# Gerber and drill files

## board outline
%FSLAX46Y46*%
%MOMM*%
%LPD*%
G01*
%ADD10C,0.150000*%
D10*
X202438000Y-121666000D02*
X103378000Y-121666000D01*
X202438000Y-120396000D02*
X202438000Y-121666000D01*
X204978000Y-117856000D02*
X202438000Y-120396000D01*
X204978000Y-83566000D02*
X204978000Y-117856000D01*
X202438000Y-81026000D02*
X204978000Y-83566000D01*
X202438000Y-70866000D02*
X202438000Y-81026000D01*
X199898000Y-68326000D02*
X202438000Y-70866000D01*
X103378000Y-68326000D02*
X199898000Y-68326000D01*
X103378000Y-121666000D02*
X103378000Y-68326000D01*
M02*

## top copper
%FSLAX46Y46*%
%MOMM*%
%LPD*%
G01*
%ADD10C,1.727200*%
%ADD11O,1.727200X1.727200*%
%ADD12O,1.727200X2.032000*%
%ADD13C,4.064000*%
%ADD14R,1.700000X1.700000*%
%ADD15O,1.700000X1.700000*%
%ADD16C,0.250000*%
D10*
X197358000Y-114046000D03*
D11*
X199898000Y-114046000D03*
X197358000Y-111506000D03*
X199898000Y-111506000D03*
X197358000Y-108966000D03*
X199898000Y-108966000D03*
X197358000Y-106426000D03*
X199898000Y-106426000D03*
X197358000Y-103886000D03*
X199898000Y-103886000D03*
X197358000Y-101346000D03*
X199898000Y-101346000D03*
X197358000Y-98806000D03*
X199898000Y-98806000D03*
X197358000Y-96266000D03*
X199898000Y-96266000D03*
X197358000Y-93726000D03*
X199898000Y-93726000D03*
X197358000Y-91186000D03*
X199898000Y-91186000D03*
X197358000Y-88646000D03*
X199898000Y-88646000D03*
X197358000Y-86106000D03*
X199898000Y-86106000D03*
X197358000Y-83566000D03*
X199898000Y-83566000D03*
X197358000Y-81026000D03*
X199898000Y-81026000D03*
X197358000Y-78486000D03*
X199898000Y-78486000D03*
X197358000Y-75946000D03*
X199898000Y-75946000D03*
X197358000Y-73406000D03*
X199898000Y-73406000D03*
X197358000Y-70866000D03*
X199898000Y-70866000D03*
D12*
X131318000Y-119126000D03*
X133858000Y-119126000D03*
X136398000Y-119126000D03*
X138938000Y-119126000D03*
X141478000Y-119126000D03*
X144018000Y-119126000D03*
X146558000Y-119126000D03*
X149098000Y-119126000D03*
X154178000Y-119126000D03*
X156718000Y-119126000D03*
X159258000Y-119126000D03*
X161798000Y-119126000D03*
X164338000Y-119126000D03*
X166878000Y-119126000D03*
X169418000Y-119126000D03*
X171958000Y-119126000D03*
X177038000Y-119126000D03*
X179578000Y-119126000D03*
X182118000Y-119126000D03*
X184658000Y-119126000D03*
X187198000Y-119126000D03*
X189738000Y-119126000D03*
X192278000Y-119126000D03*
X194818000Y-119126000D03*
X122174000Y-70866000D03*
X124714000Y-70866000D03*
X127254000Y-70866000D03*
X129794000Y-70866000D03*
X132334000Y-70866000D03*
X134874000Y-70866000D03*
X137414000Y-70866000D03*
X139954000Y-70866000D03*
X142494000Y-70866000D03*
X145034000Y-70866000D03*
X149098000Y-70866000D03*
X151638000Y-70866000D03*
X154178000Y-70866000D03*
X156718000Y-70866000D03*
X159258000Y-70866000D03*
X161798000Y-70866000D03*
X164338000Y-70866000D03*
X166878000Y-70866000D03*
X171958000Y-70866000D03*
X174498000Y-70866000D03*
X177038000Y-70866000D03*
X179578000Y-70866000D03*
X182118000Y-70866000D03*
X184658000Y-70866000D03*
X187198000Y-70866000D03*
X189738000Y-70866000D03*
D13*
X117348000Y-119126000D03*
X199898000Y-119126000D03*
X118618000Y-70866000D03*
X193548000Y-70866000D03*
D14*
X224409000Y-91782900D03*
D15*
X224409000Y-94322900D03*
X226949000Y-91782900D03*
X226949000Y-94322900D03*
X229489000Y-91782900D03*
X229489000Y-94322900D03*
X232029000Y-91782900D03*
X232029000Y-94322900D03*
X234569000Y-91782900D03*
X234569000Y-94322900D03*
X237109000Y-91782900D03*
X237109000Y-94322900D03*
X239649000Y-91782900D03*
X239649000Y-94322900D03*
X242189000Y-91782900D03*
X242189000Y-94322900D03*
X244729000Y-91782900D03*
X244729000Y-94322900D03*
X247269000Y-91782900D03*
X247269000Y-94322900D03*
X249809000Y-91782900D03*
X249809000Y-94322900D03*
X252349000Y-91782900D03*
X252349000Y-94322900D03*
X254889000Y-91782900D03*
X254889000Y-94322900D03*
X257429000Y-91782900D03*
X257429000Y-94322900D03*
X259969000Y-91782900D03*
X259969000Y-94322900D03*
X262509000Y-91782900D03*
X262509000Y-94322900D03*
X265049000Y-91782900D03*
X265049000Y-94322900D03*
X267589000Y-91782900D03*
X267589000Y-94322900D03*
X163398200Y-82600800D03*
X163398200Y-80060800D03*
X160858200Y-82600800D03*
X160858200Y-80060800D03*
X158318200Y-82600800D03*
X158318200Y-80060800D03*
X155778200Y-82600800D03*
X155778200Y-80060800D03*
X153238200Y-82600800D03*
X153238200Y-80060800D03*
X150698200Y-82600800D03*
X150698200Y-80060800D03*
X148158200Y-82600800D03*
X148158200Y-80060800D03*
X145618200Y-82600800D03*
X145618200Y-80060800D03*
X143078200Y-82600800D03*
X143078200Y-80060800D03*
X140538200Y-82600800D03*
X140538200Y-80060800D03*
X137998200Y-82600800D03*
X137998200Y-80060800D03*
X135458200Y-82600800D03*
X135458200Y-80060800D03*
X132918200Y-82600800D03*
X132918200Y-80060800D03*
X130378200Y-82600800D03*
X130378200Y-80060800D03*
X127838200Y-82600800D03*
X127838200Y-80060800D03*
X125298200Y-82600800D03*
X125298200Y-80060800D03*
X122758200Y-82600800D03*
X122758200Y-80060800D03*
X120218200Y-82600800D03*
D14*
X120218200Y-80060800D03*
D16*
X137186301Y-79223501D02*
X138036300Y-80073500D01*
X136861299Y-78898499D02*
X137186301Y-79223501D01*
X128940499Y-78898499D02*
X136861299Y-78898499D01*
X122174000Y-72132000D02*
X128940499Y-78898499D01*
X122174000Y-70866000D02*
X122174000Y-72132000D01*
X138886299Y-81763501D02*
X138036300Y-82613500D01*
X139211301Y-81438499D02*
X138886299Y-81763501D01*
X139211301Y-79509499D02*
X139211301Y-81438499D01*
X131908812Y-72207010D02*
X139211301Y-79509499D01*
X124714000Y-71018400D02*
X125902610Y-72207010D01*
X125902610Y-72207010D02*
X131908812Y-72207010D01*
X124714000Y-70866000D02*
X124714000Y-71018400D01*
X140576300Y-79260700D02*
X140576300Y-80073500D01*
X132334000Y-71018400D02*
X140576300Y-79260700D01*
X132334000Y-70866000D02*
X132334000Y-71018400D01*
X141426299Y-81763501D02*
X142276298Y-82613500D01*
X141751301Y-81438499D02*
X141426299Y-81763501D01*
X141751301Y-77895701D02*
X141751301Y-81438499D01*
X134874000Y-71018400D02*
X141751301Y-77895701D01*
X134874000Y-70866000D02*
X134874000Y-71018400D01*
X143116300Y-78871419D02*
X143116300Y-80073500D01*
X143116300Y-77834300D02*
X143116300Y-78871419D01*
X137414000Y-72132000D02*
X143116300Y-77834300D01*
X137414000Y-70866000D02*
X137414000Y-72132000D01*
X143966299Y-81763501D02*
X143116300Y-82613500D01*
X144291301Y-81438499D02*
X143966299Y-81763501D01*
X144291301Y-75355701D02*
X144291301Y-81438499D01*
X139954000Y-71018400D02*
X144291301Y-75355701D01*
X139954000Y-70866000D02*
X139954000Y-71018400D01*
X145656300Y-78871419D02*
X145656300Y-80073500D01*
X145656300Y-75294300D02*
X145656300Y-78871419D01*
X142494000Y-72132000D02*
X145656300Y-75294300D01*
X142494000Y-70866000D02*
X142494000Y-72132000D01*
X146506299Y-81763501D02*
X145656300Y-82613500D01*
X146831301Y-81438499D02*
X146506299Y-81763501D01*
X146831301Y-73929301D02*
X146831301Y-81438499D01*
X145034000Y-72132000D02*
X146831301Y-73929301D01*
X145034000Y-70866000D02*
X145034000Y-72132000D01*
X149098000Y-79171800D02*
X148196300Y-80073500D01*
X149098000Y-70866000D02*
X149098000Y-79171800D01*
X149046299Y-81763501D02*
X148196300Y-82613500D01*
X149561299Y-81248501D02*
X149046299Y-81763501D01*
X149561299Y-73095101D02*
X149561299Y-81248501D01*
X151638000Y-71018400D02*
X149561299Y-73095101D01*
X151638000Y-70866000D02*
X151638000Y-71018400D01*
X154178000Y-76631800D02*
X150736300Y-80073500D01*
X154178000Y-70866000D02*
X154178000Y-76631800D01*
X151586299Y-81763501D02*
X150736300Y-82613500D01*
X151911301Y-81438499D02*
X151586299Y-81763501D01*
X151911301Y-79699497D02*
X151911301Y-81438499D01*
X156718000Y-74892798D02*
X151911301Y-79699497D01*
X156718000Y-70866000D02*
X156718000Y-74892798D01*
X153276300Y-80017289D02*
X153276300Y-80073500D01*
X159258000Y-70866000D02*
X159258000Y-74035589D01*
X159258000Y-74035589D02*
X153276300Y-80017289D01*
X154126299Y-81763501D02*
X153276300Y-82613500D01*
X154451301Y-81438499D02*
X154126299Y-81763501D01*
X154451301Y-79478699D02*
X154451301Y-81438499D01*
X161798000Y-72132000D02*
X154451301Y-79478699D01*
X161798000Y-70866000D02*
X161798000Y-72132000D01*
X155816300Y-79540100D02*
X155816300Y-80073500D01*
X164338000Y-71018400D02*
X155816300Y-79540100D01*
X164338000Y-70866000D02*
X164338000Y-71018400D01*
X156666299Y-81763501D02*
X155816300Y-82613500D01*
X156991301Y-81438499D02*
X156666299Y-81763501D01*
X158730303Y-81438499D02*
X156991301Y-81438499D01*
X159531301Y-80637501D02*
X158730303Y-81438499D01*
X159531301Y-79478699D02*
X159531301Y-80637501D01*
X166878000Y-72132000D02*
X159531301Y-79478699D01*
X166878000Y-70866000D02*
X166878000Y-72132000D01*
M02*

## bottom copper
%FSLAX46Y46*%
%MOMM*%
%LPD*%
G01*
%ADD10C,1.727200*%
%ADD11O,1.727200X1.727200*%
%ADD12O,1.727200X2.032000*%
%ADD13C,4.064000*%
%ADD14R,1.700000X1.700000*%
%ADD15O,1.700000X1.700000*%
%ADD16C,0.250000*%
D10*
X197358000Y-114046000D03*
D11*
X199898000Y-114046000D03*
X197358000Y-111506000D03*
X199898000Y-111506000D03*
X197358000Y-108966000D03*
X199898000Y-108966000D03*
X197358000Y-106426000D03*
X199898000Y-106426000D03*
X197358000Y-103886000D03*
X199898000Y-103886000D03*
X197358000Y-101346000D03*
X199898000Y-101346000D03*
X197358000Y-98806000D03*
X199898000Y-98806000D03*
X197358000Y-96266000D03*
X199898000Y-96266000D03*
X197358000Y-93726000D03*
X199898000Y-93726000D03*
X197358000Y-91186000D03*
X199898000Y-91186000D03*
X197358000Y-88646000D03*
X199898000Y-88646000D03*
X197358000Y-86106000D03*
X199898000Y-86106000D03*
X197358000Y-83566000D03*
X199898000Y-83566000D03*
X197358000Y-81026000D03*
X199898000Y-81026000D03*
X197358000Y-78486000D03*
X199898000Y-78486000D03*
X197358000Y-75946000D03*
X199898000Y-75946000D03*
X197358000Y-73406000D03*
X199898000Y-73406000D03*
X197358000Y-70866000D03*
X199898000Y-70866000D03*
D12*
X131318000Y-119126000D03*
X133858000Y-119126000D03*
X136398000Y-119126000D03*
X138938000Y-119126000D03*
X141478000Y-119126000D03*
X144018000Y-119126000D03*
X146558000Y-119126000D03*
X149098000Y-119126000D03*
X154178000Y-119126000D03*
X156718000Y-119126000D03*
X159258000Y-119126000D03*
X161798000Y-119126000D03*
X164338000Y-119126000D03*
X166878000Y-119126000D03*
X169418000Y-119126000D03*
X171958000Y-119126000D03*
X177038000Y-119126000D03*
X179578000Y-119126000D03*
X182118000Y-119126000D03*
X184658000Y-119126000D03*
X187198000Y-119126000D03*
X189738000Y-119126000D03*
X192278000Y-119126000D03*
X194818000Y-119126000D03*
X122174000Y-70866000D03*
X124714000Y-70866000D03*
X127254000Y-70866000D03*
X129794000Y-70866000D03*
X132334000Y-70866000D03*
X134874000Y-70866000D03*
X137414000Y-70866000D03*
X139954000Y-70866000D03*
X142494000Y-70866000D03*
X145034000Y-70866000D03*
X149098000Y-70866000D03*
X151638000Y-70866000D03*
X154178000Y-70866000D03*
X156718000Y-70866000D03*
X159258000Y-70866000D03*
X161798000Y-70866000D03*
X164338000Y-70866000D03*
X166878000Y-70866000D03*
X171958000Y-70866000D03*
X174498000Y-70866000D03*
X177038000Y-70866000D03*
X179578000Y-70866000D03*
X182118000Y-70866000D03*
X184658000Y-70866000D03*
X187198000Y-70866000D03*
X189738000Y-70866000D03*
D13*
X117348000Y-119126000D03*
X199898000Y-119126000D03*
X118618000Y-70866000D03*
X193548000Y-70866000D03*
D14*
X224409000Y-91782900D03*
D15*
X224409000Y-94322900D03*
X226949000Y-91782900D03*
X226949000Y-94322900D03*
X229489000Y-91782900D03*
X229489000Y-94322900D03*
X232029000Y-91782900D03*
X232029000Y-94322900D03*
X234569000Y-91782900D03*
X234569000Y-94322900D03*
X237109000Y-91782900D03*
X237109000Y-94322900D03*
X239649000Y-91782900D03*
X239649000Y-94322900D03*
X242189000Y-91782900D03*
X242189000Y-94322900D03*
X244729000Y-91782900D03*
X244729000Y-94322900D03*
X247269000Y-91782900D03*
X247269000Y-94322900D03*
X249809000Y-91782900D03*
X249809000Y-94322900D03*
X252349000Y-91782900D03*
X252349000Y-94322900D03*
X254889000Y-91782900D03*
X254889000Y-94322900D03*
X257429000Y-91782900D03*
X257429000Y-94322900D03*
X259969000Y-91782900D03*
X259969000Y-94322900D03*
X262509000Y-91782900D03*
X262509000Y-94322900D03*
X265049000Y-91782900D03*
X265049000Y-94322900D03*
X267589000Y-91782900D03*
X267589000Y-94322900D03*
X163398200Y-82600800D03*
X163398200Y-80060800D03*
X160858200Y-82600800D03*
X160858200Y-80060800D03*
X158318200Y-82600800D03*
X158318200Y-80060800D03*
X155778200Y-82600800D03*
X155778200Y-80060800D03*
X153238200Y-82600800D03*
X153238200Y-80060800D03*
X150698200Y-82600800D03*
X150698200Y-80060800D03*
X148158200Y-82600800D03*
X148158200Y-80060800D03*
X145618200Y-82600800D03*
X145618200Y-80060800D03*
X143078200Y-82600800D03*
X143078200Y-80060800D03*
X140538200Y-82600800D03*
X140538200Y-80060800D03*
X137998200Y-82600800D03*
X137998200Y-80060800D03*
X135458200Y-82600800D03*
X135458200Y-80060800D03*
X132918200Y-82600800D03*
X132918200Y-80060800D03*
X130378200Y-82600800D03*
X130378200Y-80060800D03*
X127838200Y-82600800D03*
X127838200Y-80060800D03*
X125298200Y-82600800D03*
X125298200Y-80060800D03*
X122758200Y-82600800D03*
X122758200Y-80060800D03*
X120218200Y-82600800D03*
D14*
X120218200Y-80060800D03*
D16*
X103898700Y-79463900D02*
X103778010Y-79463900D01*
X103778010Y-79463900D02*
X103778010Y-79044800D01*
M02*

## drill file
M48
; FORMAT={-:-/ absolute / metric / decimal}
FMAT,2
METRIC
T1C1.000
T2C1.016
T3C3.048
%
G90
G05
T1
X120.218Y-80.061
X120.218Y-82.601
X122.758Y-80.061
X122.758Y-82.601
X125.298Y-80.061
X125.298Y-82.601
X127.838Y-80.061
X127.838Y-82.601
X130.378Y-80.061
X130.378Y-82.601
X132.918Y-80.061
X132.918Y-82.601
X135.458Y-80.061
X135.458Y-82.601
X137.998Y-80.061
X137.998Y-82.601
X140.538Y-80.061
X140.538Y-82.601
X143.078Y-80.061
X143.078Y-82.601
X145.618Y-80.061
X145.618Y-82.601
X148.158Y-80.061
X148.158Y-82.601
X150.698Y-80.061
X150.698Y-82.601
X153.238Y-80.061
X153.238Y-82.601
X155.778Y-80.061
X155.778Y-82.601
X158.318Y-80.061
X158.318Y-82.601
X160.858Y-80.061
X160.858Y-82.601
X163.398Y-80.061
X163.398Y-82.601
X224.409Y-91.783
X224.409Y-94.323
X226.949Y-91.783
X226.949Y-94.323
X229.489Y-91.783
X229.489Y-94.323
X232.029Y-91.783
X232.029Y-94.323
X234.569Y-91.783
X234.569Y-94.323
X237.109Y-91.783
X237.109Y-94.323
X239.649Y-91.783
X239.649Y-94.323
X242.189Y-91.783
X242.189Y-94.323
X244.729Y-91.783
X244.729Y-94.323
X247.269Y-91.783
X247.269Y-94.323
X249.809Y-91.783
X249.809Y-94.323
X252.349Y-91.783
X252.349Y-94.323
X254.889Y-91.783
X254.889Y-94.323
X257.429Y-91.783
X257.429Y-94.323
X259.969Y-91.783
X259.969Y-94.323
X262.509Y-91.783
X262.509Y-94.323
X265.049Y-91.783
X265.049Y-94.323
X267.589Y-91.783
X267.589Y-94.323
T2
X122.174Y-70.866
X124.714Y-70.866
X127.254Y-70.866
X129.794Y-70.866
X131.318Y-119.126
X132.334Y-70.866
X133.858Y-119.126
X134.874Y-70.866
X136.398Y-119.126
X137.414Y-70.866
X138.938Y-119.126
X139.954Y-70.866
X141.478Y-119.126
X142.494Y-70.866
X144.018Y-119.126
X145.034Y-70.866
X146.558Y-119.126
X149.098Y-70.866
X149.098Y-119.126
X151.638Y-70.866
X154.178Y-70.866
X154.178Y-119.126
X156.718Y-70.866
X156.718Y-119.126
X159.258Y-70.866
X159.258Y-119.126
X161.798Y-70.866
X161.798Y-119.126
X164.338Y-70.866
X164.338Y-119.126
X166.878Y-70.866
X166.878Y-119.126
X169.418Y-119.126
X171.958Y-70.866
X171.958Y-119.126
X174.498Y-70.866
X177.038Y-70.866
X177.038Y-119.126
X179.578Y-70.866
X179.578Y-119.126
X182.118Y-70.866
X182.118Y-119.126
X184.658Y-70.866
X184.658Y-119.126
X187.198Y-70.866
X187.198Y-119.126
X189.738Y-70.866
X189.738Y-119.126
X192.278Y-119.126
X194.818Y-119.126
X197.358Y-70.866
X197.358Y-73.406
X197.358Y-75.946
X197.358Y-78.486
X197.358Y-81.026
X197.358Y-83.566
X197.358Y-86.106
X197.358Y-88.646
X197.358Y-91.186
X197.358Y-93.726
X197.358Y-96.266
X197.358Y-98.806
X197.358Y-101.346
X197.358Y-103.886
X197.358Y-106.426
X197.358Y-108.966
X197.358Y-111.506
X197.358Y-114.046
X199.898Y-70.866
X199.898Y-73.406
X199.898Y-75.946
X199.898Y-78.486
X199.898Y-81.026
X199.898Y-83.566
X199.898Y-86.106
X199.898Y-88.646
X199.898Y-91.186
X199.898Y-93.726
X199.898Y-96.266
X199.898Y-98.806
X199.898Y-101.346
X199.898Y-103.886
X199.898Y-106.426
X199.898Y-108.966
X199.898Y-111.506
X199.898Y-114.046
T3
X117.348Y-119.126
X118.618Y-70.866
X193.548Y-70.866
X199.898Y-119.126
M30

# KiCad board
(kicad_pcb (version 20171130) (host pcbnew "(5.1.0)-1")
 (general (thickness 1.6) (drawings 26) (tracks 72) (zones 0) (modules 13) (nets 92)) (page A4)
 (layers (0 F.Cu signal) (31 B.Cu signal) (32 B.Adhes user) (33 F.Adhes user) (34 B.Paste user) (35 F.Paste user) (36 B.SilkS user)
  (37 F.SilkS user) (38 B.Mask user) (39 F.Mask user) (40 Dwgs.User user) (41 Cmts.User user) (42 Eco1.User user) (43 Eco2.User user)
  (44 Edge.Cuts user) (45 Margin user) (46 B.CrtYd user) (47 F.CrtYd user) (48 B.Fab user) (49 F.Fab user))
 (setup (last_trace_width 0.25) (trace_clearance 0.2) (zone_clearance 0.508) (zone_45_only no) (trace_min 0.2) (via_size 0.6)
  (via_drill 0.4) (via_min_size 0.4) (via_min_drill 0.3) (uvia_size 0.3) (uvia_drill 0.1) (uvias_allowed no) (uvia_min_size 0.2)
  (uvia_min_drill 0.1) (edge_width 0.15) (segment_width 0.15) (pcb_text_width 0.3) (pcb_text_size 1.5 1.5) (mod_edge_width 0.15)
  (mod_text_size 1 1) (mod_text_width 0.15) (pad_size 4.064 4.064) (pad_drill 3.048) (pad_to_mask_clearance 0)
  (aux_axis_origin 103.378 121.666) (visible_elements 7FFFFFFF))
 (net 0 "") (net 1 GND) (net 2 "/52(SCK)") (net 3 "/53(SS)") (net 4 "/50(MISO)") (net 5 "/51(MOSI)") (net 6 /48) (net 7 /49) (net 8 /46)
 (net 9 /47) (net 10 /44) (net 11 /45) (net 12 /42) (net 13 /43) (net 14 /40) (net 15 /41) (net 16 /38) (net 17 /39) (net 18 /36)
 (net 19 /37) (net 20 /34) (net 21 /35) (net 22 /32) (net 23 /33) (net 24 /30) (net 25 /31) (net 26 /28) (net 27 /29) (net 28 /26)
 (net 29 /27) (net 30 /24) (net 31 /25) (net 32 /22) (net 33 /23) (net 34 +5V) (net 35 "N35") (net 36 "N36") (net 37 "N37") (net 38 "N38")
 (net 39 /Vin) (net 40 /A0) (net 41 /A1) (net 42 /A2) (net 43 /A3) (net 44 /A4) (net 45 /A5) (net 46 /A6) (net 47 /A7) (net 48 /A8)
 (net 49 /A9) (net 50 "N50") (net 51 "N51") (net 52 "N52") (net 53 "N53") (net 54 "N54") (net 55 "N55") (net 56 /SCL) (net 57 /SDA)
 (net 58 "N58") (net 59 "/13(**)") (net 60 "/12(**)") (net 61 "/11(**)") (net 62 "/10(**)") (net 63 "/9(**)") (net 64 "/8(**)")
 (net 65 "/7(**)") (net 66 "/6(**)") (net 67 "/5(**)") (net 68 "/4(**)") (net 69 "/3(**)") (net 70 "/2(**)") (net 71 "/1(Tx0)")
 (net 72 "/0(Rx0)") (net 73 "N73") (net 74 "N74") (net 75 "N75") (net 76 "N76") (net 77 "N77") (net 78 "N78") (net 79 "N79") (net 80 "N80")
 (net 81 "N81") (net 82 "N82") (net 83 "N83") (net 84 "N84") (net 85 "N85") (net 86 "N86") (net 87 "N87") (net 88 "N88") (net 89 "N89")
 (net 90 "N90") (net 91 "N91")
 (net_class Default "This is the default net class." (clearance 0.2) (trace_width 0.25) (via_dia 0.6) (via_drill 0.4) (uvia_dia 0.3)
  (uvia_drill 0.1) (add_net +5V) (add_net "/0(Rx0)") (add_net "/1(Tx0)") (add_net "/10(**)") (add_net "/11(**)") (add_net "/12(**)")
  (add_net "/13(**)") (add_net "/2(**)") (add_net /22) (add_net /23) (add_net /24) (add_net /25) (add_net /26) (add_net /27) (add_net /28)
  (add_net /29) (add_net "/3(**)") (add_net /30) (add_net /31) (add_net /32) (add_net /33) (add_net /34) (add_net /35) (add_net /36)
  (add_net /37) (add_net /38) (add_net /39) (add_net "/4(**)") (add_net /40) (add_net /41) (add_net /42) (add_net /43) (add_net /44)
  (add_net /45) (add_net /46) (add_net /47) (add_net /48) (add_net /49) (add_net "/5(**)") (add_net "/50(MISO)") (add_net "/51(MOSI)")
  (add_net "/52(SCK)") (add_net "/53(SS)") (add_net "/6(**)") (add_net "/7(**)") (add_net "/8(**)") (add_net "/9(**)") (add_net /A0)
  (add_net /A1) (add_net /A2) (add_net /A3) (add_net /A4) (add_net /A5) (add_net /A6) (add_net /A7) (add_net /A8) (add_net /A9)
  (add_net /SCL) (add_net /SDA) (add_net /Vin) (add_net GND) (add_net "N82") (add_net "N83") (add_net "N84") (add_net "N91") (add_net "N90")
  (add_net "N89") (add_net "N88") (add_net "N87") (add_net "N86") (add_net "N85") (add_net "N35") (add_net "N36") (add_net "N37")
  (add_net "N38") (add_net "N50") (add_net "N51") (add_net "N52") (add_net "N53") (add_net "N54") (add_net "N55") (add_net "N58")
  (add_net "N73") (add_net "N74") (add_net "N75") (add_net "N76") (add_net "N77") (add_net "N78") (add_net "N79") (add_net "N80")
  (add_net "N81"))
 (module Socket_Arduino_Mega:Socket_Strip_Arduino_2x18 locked (layer F.Cu) (at 197.358 114.046 90)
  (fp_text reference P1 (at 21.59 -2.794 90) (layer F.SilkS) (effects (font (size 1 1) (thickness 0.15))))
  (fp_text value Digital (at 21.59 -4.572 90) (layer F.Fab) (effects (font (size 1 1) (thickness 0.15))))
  (pad 1 thru_hole circle (at 0 0 90) (size 1.7272 1.7272) (drill 1.016) (layers *.Cu *.Mask F.SilkS) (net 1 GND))
  (pad 2 thru_hole oval (at 0 2.54 90) (size 1.7272 1.7272) (drill 1.016) (layers *.Cu *.Mask F.SilkS) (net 1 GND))
  (pad 3 thru_hole oval (at 2.54 0 90) (size 1.7272 1.7272) (drill 1.016) (layers *.Cu *.Mask F.SilkS) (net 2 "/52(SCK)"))
  (pad 4 thru_hole oval (at 2.54 2.54 90) (size 1.7272 1.7272) (drill 1.016) (layers *.Cu *.Mask F.SilkS) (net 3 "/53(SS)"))
  (pad 5 thru_hole oval (at 5.08 0 90) (size 1.7272 1.7272) (drill 1.016) (layers *.Cu *.Mask F.SilkS) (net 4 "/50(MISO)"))
  (pad 6 thru_hole oval (at 5.08 2.54 90) (size 1.7272 1.7272) (drill 1.016) (layers *.Cu *.Mask F.SilkS) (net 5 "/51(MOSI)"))
  (pad 7 thru_hole oval (at 7.62 0 90) (size 1.7272 1.7272) (drill 1.016) (layers *.Cu *.Mask F.SilkS) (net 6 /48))
  (pad 8 thru_hole oval (at 7.62 2.54 90) (size 1.7272 1.7272) (drill 1.016) (layers *.Cu *.Mask F.SilkS) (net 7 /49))
  (pad 9 thru_hole oval (at 10.16 0 90) (size 1.7272 1.7272) (drill 1.016) (layers *.Cu *.Mask F.SilkS) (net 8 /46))
  (pad 10 thru_hole oval (at 10.16 2.54 90) (size 1.7272 1.7272) (drill 1.016) (layers *.Cu *.Mask F.SilkS) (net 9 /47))
  (pad 11 thru_hole oval (at 12.7 0 90) (size 1.7272 1.7272) (drill 1.016) (layers *.Cu *.Mask F.SilkS) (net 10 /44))
  (pad 12 thru_hole oval (at 12.7 2.54 90) (size 1.7272 1.7272) (drill 1.016) (layers *.Cu *.Mask F.SilkS) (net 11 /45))
  (pad 13 thru_hole oval (at 15.24 0 90) (size 1.7272 1.7272) (drill 1.016) (layers *.Cu *.Mask F.SilkS) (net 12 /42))
  (pad 14 thru_hole oval (at 15.24 2.54 90) (size 1.7272 1.7272) (drill 1.016) (layers *.Cu *.Mask F.SilkS) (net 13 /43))
  (pad 15 thru_hole oval (at 17.78 0 90) (size 1.7272 1.7272) (drill 1.016) (layers *.Cu *.Mask F.SilkS) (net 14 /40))
  (pad 16 thru_hole oval (at 17.78 2.54 90) (size 1.7272 1.7272) (drill 1.016) (layers *.Cu *.Mask F.SilkS) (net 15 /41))
  (pad 17 thru_hole oval (at 20.32 0 90) (size 1.7272 1.7272) (drill 1.016) (layers *.Cu *.Mask F.SilkS) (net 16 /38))
  (pad 18 thru_hole oval (at 20.32 2.54 90) (size 1.7272 1.7272) (drill 1.016) (layers *.Cu *.Mask F.SilkS) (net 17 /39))
  (pad 19 thru_hole oval (at 22.86 0 90) (size 1.7272 1.7272) (drill 1.016) (layers *.Cu *.Mask F.SilkS) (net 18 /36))
  (pad 20 thru_hole oval (at 22.86 2.54 90) (size 1.7272 1.7272) (drill 1.016) (layers *.Cu *.Mask F.SilkS) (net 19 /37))
  (pad 21 thru_hole oval (at 25.4 0 90) (size 1.7272 1.7272) (drill 1.016) (layers *.Cu *.Mask F.SilkS) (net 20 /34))
  (pad 22 thru_hole oval (at 25.4 2.54 90) (size 1.7272 1.7272) (drill 1.016) (layers *.Cu *.Mask F.SilkS) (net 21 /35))
  (pad 23 thru_hole oval (at 27.94 0 90) (size 1.7272 1.7272) (drill 1.016) (layers *.Cu *.Mask F.SilkS) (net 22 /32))
  (pad 24 thru_hole oval (at 27.94 2.54 90) (size 1.7272 1.7272) (drill 1.016) (layers *.Cu *.Mask F.SilkS) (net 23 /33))
  (pad 25 thru_hole oval (at 30.48 0 90) (size 1.7272 1.7272) (drill 1.016) (layers *.Cu *.Mask F.SilkS) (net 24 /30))
  (pad 26 thru_hole oval (at 30.48 2.54 90) (size 1.7272 1.7272) (drill 1.016) (layers *.Cu *.Mask F.SilkS) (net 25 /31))
  (pad 27 thru_hole oval (at 33.02 0 90) (size 1.7272 1.7272) (drill 1.016) (layers *.Cu *.Mask F.SilkS) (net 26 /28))
  (pad 28 thru_hole oval (at 33.02 2.54 90) (size 1.7272 1.7272) (drill 1.016) (layers *.Cu *.Mask F.SilkS) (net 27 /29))
  (pad 29 thru_hole oval (at 35.56 0 90) (size 1.7272 1.7272) (drill 1.016) (layers *.Cu *.Mask F.SilkS) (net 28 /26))
  (pad 30 thru_hole oval (at 35.56 2.54 90) (size 1.7272 1.7272) (drill 1.016) (layers *.Cu *.Mask F.SilkS) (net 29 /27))
  (pad 31 thru_hole oval (at 38.1 0 90) (size 1.7272 1.7272) (drill 1.016) (layers *.Cu *.Mask F.SilkS) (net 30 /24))
  (pad 32 thru_hole oval (at 38.1 2.54 90) (size 1.7272 1.7272) (drill 1.016) (layers *.Cu *.Mask F.SilkS) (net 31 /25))
  (pad 33 thru_hole oval (at 40.64 0 90) (size 1.7272 1.7272) (drill 1.016) (layers *.Cu *.Mask F.SilkS) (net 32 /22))
  (pad 34 thru_hole oval (at 40.64 2.54 90) (size 1.7272 1.7272) (drill 1.016) (layers *.Cu *.Mask F.SilkS) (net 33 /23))
  (pad 35 thru_hole oval (at 43.18 0 90) (size 1.7272 1.7272) (drill 1.016) (layers *.Cu *.Mask F.SilkS) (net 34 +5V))
  (pad 36 thru_hole oval (at 43.18 2.54 90) (size 1.7272 1.7272) (drill 1.016) (layers *.Cu *.Mask F.SilkS) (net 34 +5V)))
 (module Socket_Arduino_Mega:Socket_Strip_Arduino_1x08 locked (layer F.Cu) (at 131.318 119.126)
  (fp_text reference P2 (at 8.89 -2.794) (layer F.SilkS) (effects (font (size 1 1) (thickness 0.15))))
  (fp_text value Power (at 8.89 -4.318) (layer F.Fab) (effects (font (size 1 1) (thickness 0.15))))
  (pad 1 thru_hole oval (at 0 0) (size 1.7272 2.032) (drill 1.016) (layers *.Cu *.Mask F.SilkS) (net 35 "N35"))
  (pad 2 thru_hole oval (at 2.54 0) (size 1.7272 2.032) (drill 1.016) (layers *.Cu *.Mask F.SilkS) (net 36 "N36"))
  (pad 3 thru_hole oval (at 5.08 0) (size 1.7272 2.032) (drill 1.016) (layers *.Cu *.Mask F.SilkS) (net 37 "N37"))
  (pad 4 thru_hole oval (at 7.62 0) (size 1.7272 2.032) (drill 1.016) (layers *.Cu *.Mask F.SilkS) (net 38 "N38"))
  (pad 5 thru_hole oval (at 10.16 0) (size 1.7272 2.032) (drill 1.016) (layers *.Cu *.Mask F.SilkS) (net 34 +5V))
  (pad 6 thru_hole oval (at 12.7 0) (size 1.7272 2.032) (drill 1.016) (layers *.Cu *.Mask F.SilkS) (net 1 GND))
  (pad 7 thru_hole oval (at 15.24 0) (size 1.7272 2.032) (drill 1.016) (layers *.Cu *.Mask F.SilkS) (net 1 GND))
  (pad 8 thru_hole oval (at 17.78 0) (size 1.7272 2.032) (drill 1.016) (layers *.Cu *.Mask F.SilkS) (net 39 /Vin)))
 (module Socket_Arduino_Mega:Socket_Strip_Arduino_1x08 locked (layer F.Cu) (at 154.178 119.126)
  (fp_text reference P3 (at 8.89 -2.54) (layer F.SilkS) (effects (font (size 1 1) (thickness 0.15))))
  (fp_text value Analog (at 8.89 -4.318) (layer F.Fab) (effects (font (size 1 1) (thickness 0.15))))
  (pad 1 thru_hole oval (at 0 0) (size 1.7272 2.032) (drill 1.016) (layers *.Cu *.Mask F.SilkS) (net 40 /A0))
  (pad 2 thru_hole oval (at 2.54 0) (size 1.7272 2.032) (drill 1.016) (layers *.Cu *.Mask F.SilkS) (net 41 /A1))
  (pad 3 thru_hole oval (at 5.08 0) (size 1.7272 2.032) (drill 1.016) (layers *.Cu *.Mask F.SilkS) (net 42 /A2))
  (pad 4 thru_hole oval (at 7.62 0) (size 1.7272 2.032) (drill 1.016) (layers *.Cu *.Mask F.SilkS) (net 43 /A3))
  (pad 5 thru_hole oval (at 10.16 0) (size 1.7272 2.032) (drill 1.016) (layers *.Cu *.Mask F.SilkS) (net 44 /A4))
  (pad 6 thru_hole oval (at 12.7 0) (size 1.7272 2.032) (drill 1.016) (layers *.Cu *.Mask F.SilkS) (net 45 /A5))
  (pad 7 thru_hole oval (at 15.24 0) (size 1.7272 2.032) (drill 1.016) (layers *.Cu *.Mask F.SilkS) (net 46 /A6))
  (pad 8 thru_hole oval (at 17.78 0) (size 1.7272 2.032) (drill 1.016) (layers *.Cu *.Mask F.SilkS) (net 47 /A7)))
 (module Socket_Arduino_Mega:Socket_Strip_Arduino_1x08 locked (layer F.Cu) (at 177.038 119.126)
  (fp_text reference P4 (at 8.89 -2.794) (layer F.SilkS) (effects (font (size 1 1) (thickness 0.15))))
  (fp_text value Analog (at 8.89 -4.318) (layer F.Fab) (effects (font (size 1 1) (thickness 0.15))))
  (pad 1 thru_hole oval (at 0 0) (size 1.7272 2.032) (drill 1.016) (layers *.Cu *.Mask F.SilkS) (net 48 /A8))
  (pad 2 thru_hole oval (at 2.54 0) (size 1.7272 2.032) (drill 1.016) (layers *.Cu *.Mask F.SilkS) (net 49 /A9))
  (pad 3 thru_hole oval (at 5.08 0) (size 1.7272 2.032) (drill 1.016) (layers *.Cu *.Mask F.SilkS) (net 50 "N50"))
  (pad 4 thru_hole oval (at 7.62 0) (size 1.7272 2.032) (drill 1.016) (layers *.Cu *.Mask F.SilkS) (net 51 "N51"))
  (pad 5 thru_hole oval (at 10.16 0) (size 1.7272 2.032) (drill 1.016) (layers *.Cu *.Mask F.SilkS) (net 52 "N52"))
  (pad 6 thru_hole oval (at 12.7 0) (size 1.7272 2.032) (drill 1.016) (layers *.Cu *.Mask F.SilkS) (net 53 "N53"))
  (pad 7 thru_hole oval (at 15.24 0) (size 1.7272 2.032) (drill 1.016) (layers *.Cu *.Mask F.SilkS) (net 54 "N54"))
  (pad 8 thru_hole oval (at 17.78 0) (size 1.7272 2.032) (drill 1.016) (layers *.Cu *.Mask F.SilkS) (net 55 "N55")))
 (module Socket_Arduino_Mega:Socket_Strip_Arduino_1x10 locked (layer F.Cu) (at 122.174 70.866)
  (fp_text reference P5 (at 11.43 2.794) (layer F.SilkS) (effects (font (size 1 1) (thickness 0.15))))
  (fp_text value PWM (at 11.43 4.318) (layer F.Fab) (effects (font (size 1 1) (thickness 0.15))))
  (pad 1 thru_hole oval (at 0 0) (size 1.7272 2.032) (drill 1.016) (layers *.Cu *.Mask F.SilkS) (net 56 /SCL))
  (pad 2 thru_hole oval (at 2.54 0) (size 1.7272 2.032) (drill 1.016) (layers *.Cu *.Mask F.SilkS) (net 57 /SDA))
  (pad 3 thru_hole oval (at 5.08 0) (size 1.7272 2.032) (drill 1.016) (layers *.Cu *.Mask F.SilkS) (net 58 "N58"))
  (pad 4 thru_hole oval (at 7.62 0) (size 1.7272 2.032) (drill 1.016) (layers *.Cu *.Mask F.SilkS) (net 1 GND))
  (pad 5 thru_hole oval (at 10.16 0) (size 1.7272 2.032) (drill 1.016) (layers *.Cu *.Mask F.SilkS) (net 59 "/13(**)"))
  (pad 6 thru_hole oval (at 12.7 0) (size 1.7272 2.032) (drill 1.016) (layers *.Cu *.Mask F.SilkS) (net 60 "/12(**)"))
  (pad 7 thru_hole oval (at 15.24 0) (size 1.7272 2.032) (drill 1.016) (layers *.Cu *.Mask F.SilkS) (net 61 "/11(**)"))
  (pad 8 thru_hole oval (at 17.78 0) (size 1.7272 2.032) (drill 1.016) (layers *.Cu *.Mask F.SilkS) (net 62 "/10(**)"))
  (pad 9 thru_hole oval (at 20.32 0) (size 1.7272 2.032) (drill 1.016) (layers *.Cu *.Mask F.SilkS) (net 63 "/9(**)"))
  (pad 10 thru_hole oval (at 22.86 0) (size 1.7272 2.032) (drill 1.016) (layers *.Cu *.Mask F.SilkS) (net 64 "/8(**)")))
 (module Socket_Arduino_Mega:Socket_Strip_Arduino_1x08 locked (layer F.Cu) (at 149.098 70.866)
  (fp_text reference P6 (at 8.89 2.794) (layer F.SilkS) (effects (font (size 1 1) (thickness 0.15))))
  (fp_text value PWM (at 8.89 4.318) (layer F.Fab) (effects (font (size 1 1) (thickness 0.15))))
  (pad 1 thru_hole oval (at 0 0) (size 1.7272 2.032) (drill 1.016) (layers *.Cu *.Mask F.SilkS) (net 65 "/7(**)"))
  (pad 2 thru_hole oval (at 2.54 0) (size 1.7272 2.032) (drill 1.016) (layers *.Cu *.Mask F.SilkS) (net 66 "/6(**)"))
  (pad 3 thru_hole oval (at 5.08 0) (size 1.7272 2.032) (drill 1.016) (layers *.Cu *.Mask F.SilkS) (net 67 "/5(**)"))
  (pad 4 thru_hole oval (at 7.62 0) (size 1.7272 2.032) (drill 1.016) (layers *.Cu *.Mask F.SilkS) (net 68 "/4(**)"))
  (pad 5 thru_hole oval (at 10.16 0) (size 1.7272 2.032) (drill 1.016) (layers *.Cu *.Mask F.SilkS) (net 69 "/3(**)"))
  (pad 6 thru_hole oval (at 12.7 0) (size 1.7272 2.032) (drill 1.016) (layers *.Cu *.Mask F.SilkS) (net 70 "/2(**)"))
  (pad 7 thru_hole oval (at 15.24 0) (size 1.7272 2.032) (drill 1.016) (layers *.Cu *.Mask F.SilkS) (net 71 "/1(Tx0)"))
  (pad 8 thru_hole oval (at 17.78 0) (size 1.7272 2.032) (drill 1.016) (layers *.Cu *.Mask F.SilkS) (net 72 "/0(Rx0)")))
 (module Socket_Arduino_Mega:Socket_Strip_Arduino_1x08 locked (layer F.Cu) (at 171.958 70.866)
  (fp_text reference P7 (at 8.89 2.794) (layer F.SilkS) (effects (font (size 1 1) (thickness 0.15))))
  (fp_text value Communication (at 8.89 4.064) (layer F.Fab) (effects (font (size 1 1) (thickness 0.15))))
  (pad 1 thru_hole oval (at 0 0) (size 1.7272 2.032) (drill 1.016) (layers *.Cu *.Mask F.SilkS) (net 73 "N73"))
  (pad 2 thru_hole oval (at 2.54 0) (size 1.7272 2.032) (drill 1.016) (layers *.Cu *.Mask F.SilkS) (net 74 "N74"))
  (pad 3 thru_hole oval (at 5.08 0) (size 1.7272 2.032) (drill 1.016) (layers *.Cu *.Mask F.SilkS) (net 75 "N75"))
  (pad 4 thru_hole oval (at 7.62 0) (size 1.7272 2.032) (drill 1.016) (layers *.Cu *.Mask F.SilkS) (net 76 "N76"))
  (pad 5 thru_hole oval (at 10.16 0) (size 1.7272 2.032) (drill 1.016) (layers *.Cu *.Mask F.SilkS) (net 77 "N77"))
  (pad 6 thru_hole oval (at 12.7 0) (size 1.7272 2.032) (drill 1.016) (layers *.Cu *.Mask F.SilkS) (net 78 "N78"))
  (pad 7 thru_hole oval (at 15.24 0) (size 1.7272 2.032) (drill 1.016) (layers *.Cu *.Mask F.SilkS) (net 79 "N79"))
  (pad 8 thru_hole oval (at 17.78 0) (size 1.7272 2.032) (drill 1.016) (layers *.Cu *.Mask F.SilkS) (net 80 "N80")))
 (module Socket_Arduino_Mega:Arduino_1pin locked (layer F.Cu) (at 117.348 119.126)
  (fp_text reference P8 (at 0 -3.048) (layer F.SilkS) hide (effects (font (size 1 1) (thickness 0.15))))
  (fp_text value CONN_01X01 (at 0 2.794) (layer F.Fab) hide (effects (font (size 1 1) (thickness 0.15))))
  (pad 1 thru_hole circle (at 0 0) (size 4.064 4.064) (drill 3.048) (layers *.Cu *.Mask F.SilkS) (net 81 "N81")))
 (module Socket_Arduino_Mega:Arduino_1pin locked (layer F.Cu) (at 199.898 119.126)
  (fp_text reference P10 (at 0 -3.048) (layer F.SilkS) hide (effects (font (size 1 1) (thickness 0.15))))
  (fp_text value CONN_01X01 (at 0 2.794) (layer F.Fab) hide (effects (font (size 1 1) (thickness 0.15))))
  (pad 1 thru_hole circle (at 0 0) (size 4.064 4.064) (drill 3.048) (layers *.Cu *.Mask F.SilkS) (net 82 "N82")))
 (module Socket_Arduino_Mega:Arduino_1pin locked (layer F.Cu) (at 118.618 70.866)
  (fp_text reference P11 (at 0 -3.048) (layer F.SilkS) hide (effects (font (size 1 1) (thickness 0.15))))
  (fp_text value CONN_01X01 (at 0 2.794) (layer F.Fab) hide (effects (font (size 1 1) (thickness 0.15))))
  (pad 1 thru_hole circle (at 0 0) (size 4.064 4.064) (drill 3.048) (layers *.Cu *.Mask F.SilkS) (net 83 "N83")))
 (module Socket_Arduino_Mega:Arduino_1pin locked (layer F.Cu) (at 193.548 70.866)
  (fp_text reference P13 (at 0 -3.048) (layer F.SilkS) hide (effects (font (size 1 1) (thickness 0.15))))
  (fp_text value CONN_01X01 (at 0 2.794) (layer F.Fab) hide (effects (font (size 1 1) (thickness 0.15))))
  (pad 1 thru_hole circle (at 0 0) (size 4.064 4.064) (drill 3.048) (layers *.Cu *.Mask F.SilkS) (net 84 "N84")))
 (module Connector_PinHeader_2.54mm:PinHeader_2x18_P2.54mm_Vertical (layer B.Cu) (at 224.409 91.7829 270)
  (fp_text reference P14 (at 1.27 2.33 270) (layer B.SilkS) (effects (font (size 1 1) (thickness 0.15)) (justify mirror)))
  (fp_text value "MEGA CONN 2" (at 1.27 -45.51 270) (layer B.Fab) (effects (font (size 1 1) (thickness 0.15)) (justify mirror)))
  (pad 1 thru_hole rect (at 0 0 270) (size 1.7 1.7) (drill 1) (layers *.Cu *.Mask) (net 1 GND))
  (pad 2 thru_hole oval (at 2.54 0 270) (size 1.7 1.7) (drill 1) (layers *.Cu *.Mask) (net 1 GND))
  (pad 3 thru_hole oval (at 0 -2.54 270) (size 1.7 1.7) (drill 1) (layers *.Cu *.Mask) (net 2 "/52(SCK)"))
  (pad 4 thru_hole oval (at 2.54 -2.54 270) (size 1.7 1.7) (drill 1) (layers *.Cu *.Mask) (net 3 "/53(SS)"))
  (pad 5 thru_hole oval (at 0 -5.08 270) (size 1.7 1.7) (drill 1) (layers *.Cu *.Mask) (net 4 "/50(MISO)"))
  (pad 6 thru_hole oval (at 2.54 -5.08 270) (size 1.7 1.7) (drill 1) (layers *.Cu *.Mask) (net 5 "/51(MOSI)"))
  (pad 7 thru_hole oval (at 0 -7.62 270) (size 1.7 1.7) (drill 1) (layers *.Cu *.Mask) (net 6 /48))
  (pad 8 thru_hole oval (at 2.54 -7.62 270) (size 1.7 1.7) (drill 1) (layers *.Cu *.Mask) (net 7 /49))
  (pad 9 thru_hole oval (at 0 -10.16 270) (size 1.7 1.7) (drill 1) (layers *.Cu *.Mask) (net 8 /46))
  (pad 10 thru_hole oval (at 2.54 -10.16 270) (size 1.7 1.7) (drill 1) (layers *.Cu *.Mask) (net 9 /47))
  (pad 11 thru_hole oval (at 0 -12.7 270) (size 1.7 1.7) (drill 1) (layers *.Cu *.Mask) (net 10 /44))
  (pad 12 thru_hole oval (at 2.54 -12.7 270) (size 1.7 1.7) (drill 1) (layers *.Cu *.Mask) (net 11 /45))
  (pad 13 thru_hole oval (at 0 -15.24 270) (size 1.7 1.7) (drill 1) (layers *.Cu *.Mask) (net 12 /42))
  (pad 14 thru_hole oval (at 2.54 -15.24 270) (size 1.7 1.7) (drill 1) (layers *.Cu *.Mask) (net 13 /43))
  (pad 15 thru_hole oval (at 0 -17.78 270) (size 1.7 1.7) (drill 1) (layers *.Cu *.Mask) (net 14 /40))
  (pad 16 thru_hole oval (at 2.54 -17.78 270) (size 1.7 1.7) (drill 1) (layers *.Cu *.Mask) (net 15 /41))
  (pad 17 thru_hole oval (at 0 -20.32 270) (size 1.7 1.7) (drill 1) (layers *.Cu *.Mask) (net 16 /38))
  (pad 18 thru_hole oval (at 2.54 -20.32 270) (size 1.7 1.7) (drill 1) (layers *.Cu *.Mask) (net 17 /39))
  (pad 19 thru_hole oval (at 0 -22.86 270) (size 1.7 1.7) (drill 1) (layers *.Cu *.Mask) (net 18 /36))
  (pad 20 thru_hole oval (at 2.54 -22.86 270) (size 1.7 1.7) (drill 1) (layers *.Cu *.Mask) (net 19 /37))
  (pad 21 thru_hole oval (at 0 -25.4 270) (size 1.7 1.7) (drill 1) (layers *.Cu *.Mask) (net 22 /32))
  (pad 22 thru_hole oval (at 2.54 -25.4 270) (size 1.7 1.7) (drill 1) (layers *.Cu *.Mask) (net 21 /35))
  (pad 23 thru_hole oval (at 0 -27.94 270) (size 1.7 1.7) (drill 1) (layers *.Cu *.Mask) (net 20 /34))
  (pad 24 thru_hole oval (at 2.54 -27.94 270) (size 1.7 1.7) (drill 1) (layers *.Cu *.Mask) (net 23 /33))
  (pad 25 thru_hole oval (at 0 -30.48 270) (size 1.7 1.7) (drill 1) (layers *.Cu *.Mask) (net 24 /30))
  (pad 26 thru_hole oval (at 2.54 -30.48 270) (size 1.7 1.7) (drill 1) (layers *.Cu *.Mask) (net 25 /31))
  (pad 27 thru_hole oval (at 0 -33.02 270) (size 1.7 1.7) (drill 1) (layers *.Cu *.Mask) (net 32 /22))
  (pad 28 thru_hole oval (at 2.54 -33.02 270) (size 1.7 1.7) (drill 1) (layers *.Cu *.Mask) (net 33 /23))
  (pad 29 thru_hole oval (at 0 -35.56 270) (size 1.7 1.7) (drill 1) (layers *.Cu *.Mask) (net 28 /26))
  (pad 30 thru_hole oval (at 2.54 -35.56 270) (size 1.7 1.7) (drill 1) (layers *.Cu *.Mask) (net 29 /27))
  (pad 31 thru_hole oval (at 0 -38.1 270) (size 1.7 1.7) (drill 1) (layers *.Cu *.Mask) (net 30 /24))
  (pad 32 thru_hole oval (at 2.54 -38.1 270) (size 1.7 1.7) (drill 1) (layers *.Cu *.Mask) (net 31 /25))
  (pad 33 thru_hole oval (at 0 -40.64 270) (size 1.7 1.7) (drill 1) (layers *.Cu *.Mask) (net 26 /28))
  (pad 34 thru_hole oval (at 2.54 -40.64 270) (size 1.7 1.7) (drill 1) (layers *.Cu *.Mask) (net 27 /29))
  (pad 35 thru_hole oval (at 0 -43.18 270) (size 1.7 1.7) (drill 1) (layers *.Cu *.Mask) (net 34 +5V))
  (pad 36 thru_hole oval (at 2.54 -43.18 270) (size 1.7 1.7) (drill 1) (layers *.Cu *.Mask) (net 34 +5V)))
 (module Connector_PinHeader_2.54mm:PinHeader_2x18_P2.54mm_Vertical (layer B.Cu) (at 120.2182 80.0608 270)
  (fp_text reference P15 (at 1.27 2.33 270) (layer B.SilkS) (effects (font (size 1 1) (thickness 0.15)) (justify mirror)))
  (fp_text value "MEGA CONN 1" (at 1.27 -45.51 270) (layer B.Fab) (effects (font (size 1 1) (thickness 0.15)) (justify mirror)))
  (pad 36 thru_hole oval (at 2.54 -43.18 270) (size 1.7 1.7) (drill 1) (layers *.Cu *.Mask) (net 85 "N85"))
  (pad 35 thru_hole oval (at 0 -43.18 270) (size 1.7 1.7) (drill 1) (layers *.Cu *.Mask) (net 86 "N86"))
  (pad 34 thru_hole oval (at 2.54 -40.64 270) (size 1.7 1.7) (drill 1) (layers *.Cu *.Mask) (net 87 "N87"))
  (pad 33 thru_hole oval (at 0 -40.64 270) (size 1.7 1.7) (drill 1) (layers *.Cu *.Mask) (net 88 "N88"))
  (pad 32 thru_hole oval (at 2.54 -38.1 270) (size 1.7 1.7) (drill 1) (layers *.Cu *.Mask) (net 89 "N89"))
  (pad 31 thru_hole oval (at 0 -38.1 270) (size 1.7 1.7) (drill 1) (layers *.Cu *.Mask) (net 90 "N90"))
  (pad 30 thru_hole oval (at 2.54 -35.56 270) (size 1.7 1.7) (drill 1) (layers *.Cu *.Mask) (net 72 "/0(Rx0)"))
  (pad 29 thru_hole oval (at 0 -35.56 270) (size 1.7 1.7) (drill 1) (layers *.Cu *.Mask) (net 71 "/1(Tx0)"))
  (pad 28 thru_hole oval (at 2.54 -33.02 270) (size 1.7 1.7) (drill 1) (layers *.Cu *.Mask) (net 70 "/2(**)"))
  (pad 27 thru_hole oval (at 0 -33.02 270) (size 1.7 1.7) (drill 1) (layers *.Cu *.Mask) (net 69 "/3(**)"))
  (pad 26 thru_hole oval (at 2.54 -30.48 270) (size 1.7 1.7) (drill 1) (layers *.Cu *.Mask) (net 68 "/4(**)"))
  (pad 25 thru_hole oval (at 0 -30.48 270) (size 1.7 1.7) (drill 1) (layers *.Cu *.Mask) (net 67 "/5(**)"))
  (pad 24 thru_hole oval (at 2.54 -27.94 270) (size 1.7 1.7) (drill 1) (layers *.Cu *.Mask) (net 66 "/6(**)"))
  (pad 23 thru_hole oval (at 0 -27.94 270) (size 1.7 1.7) (drill 1) (layers *.Cu *.Mask) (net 65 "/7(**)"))
  (pad 22 thru_hole oval (at 2.54 -25.4 270) (size 1.7 1.7) (drill 1) (layers *.Cu *.Mask) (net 64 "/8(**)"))
  (pad 21 thru_hole oval (at 0 -25.4 270) (size 1.7 1.7) (drill 1) (layers *.Cu *.Mask) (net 63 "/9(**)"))
  (pad 20 thru_hole oval (at 2.54 -22.86 270) (size 1.7 1.7) (drill 1) (layers *.Cu *.Mask) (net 62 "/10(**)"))
  (pad 19 thru_hole oval (at 0 -22.86 270) (size 1.7 1.7) (drill 1) (layers *.Cu *.Mask) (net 61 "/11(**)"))
  (pad 18 thru_hole oval (at 2.54 -20.32 270) (size 1.7 1.7) (drill 1) (layers *.Cu *.Mask) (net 60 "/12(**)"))
  (pad 17 thru_hole oval (at 0 -20.32 270) (size 1.7 1.7) (drill 1) (layers *.Cu *.Mask) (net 59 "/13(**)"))
  (pad 16 thru_hole oval (at 2.54 -17.78 270) (size 1.7 1.7) (drill 1) (layers *.Cu *.Mask) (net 57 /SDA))
  (pad 15 thru_hole oval (at 0 -17.78 270) (size 1.7 1.7) (drill 1) (layers *.Cu *.Mask) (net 56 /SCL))
  (pad 14 thru_hole oval (at 2.54 -15.24 270) (size 1.7 1.7) (drill 1) (layers *.Cu *.Mask) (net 45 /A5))
  (pad 13 thru_hole oval (at 0 -15.24 270) (size 1.7 1.7) (drill 1) (layers *.Cu *.Mask) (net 42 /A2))
  (pad 12 thru_hole oval (at 2.54 -12.7 270) (size 1.7 1.7) (drill 1) (layers *.Cu *.Mask) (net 47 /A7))
  (pad 11 thru_hole oval (at 0 -12.7 270) (size 1.7 1.7) (drill 1) (layers *.Cu *.Mask) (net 43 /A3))
  (pad 10 thru_hole oval (at 2.54 -10.16 270) (size 1.7 1.7) (drill 1) (layers *.Cu *.Mask) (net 44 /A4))
  (pad 9 thru_hole oval (at 0 -10.16 270) (size 1.7 1.7) (drill 1) (layers *.Cu *.Mask) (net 48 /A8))
  (pad 8 thru_hole oval (at 2.54 -7.62 270) (size 1.7 1.7) (drill 1) (layers *.Cu *.Mask) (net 46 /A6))
  (pad 7 thru_hole oval (at 0 -7.62 270) (size 1.7 1.7) (drill 1) (layers *.Cu *.Mask) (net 40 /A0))
  (pad 6 thru_hole oval (at 2.54 -5.08 270) (size 1.7 1.7) (drill 1) (layers *.Cu *.Mask) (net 49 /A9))
  (pad 5 thru_hole oval (at 0 -5.08 270) (size 1.7 1.7) (drill 1) (layers *.Cu *.Mask) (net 41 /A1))
  (pad 4 thru_hole oval (at 2.54 -2.54 270) (size 1.7 1.7) (drill 1) (layers *.Cu *.Mask) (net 1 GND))
  (pad 3 thru_hole oval (at 0 -2.54 270) (size 1.7 1.7) (drill 1) (layers *.Cu *.Mask) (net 39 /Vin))
  (pad 2 thru_hole oval (at 2.54 0 270) (size 1.7 1.7) (drill 1) (layers *.Cu *.Mask) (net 34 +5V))
  (pad 1 thru_hole rect (at 0 0 270) (size 1.7 1.7) (drill 1) (layers *.Cu *.Mask) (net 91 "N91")))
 (gr_line (start 202.438 121.666) (end 103.378 121.666) (angle 90) (layer Edge.Cuts) (width 0.15))
 (gr_line (start 202.438 120.396) (end 202.438 121.666) (angle 90) (layer Edge.Cuts) (width 0.15))
 (gr_line (start 204.978 117.856) (end 202.438 120.396) (angle 90) (layer Edge.Cuts) (width 0.15))
 (gr_line (start 204.978 83.566) (end 204.978 117.856) (angle 90) (layer Edge.Cuts) (width 0.15))
 (gr_line (start 202.438 81.026) (end 204.978 83.566) (angle 90) (layer Edge.Cuts) (width 0.15))
 (gr_line (start 202.438 70.866) (end 202.438 81.026) (angle 90) (layer Edge.Cuts) (width 0.15))
 (gr_line (start 199.898 68.326) (end 202.438 70.866) (angle 90) (layer Edge.Cuts) (width 0.15))
 (gr_line (start 103.378 68.326) (end 199.898 68.326) (angle 90) (layer Edge.Cuts) (width 0.15))
 (gr_line (start 103.378 121.666) (end 103.378 68.326) (angle 90) (layer Edge.Cuts) (width 0.15))
 (segment (start 103.8987 79.4639) (end 103.77801 79.4639) (width 0.25) (layer B.Cu) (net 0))
 (segment (start 103.77801 79.4639) (end 103.77801 79.0448) (width 0.25) (layer B.Cu) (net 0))
 (segment (start 137.186301 79.223501) (end 138.0363 80.0735) (width 0.25) (layer F.Cu) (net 56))
 (segment (start 136.861299 78.898499) (end 137.186301 79.223501) (width 0.25) (layer F.Cu) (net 56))
 (segment (start 128.940499 78.898499) (end 136.861299 78.898499) (width 0.25) (layer F.Cu) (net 56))
 (segment (start 122.174 72.132) (end 128.940499 78.898499) (width 0.25) (layer F.Cu) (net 56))
 (segment (start 122.174 70.866) (end 122.174 72.132) (width 0.25) (layer F.Cu) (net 56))
 (segment (start 138.886299 81.763501) (end 138.0363 82.6135) (width 0.25) (layer F.Cu) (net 57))
 (segment (start 139.211301 81.438499) (end 138.886299 81.763501) (width 0.25) (layer F.Cu) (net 57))
 (segment (start 139.211301 79.509499) (end 139.211301 81.438499) (width 0.25) (layer F.Cu) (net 57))
 (segment (start 131.908812 72.20701) (end 139.211301 79.509499) (width 0.25) (layer F.Cu) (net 57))
 (segment (start 124.714 71.0184) (end 125.90261 72.20701) (width 0.25) (layer F.Cu) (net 57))
 (segment (start 125.90261 72.20701) (end 131.908812 72.20701) (width 0.25) (layer F.Cu) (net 57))
 (segment (start 124.714 70.866) (end 124.714 71.0184) (width 0.25) (layer F.Cu) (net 57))
 (segment (start 140.5763 79.2607) (end 140.5763 80.0735) (width 0.25) (layer F.Cu) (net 59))
 (segment (start 132.334 71.0184) (end 140.5763 79.2607) (width 0.25) (layer F.Cu) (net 59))
 (segment (start 132.334 70.866) (end 132.334 71.0184) (width 0.25) (layer F.Cu) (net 59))
 (segment (start 141.426299 81.763501) (end 142.276298 82.6135) (width 0.25) (layer F.Cu) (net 60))
 (segment (start 141.751301 81.438499) (end 141.426299 81.763501) (width 0.25) (layer F.Cu) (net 60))
 (segment (start 141.751301 77.895701) (end 141.751301 81.438499) (width 0.25) (layer F.Cu) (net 60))
 (segment (start 134.874 71.0184) (end 141.751301 77.895701) (width 0.25) (layer F.Cu) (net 60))
 (segment (start 134.874 70.866) (end 134.874 71.0184) (width 0.25) (layer F.Cu) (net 60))
 (segment (start 143.1163 78.871419) (end 143.1163 80.0735) (width 0.25) (layer F.Cu) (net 61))
 (segment (start 143.1163 77.8343) (end 143.1163 78.871419) (width 0.25) (layer F.Cu) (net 61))
 (segment (start 137.414 72.132) (end 143.1163 77.8343) (width 0.25) (layer F.Cu) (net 61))
 (segment (start 137.414 70.866) (end 137.414 72.132) (width 0.25) (layer F.Cu) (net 61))
 (segment (start 143.966299 81.763501) (end 143.1163 82.6135) (width 0.25) (layer F.Cu) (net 62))
 (segment (start 144.291301 81.438499) (end 143.966299 81.763501) (width 0.25) (layer F.Cu) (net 62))
 (segment (start 144.291301 75.355701) (end 144.291301 81.438499) (width 0.25) (layer F.Cu) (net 62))
 (segment (start 139.954 71.0184) (end 144.291301 75.355701) (width 0.25) (layer F.Cu) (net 62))
 (segment (start 139.954 70.866) (end 139.954 71.0184) (width 0.25) (layer F.Cu) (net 62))
 (segment (start 145.6563 78.871419) (end 145.6563 80.0735) (width 0.25) (layer F.Cu) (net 63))
 (segment (start 145.6563 75.2943) (end 145.6563 78.871419) (width 0.25) (layer F.Cu) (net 63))
 (segment (start 142.494 72.132) (end 145.6563 75.2943) (width 0.25) (layer F.Cu) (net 63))
 (segment (start 142.494 70.866) (end 142.494 72.132) (width 0.25) (layer F.Cu) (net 63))
 (segment (start 146.506299 81.763501) (end 145.6563 82.6135) (width 0.25) (layer F.Cu) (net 64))
 (segment (start 146.831301 81.438499) (end 146.506299 81.763501) (width 0.25) (layer F.Cu) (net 64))
 (segment (start 146.831301 73.929301) (end 146.831301 81.438499) (width 0.25) (layer F.Cu) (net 64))
 (segment (start 145.034 72.132) (end 146.831301 73.929301) (width 0.25) (layer F.Cu) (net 64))
 (segment (start 145.034 70.866) (end 145.034 72.132) (width 0.25) (layer F.Cu) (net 64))
 (segment (start 149.098 79.1718) (end 148.1963 80.0735) (width 0.25) (layer F.Cu) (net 65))
 (segment (start 149.098 70.866) (end 149.098 79.1718) (width 0.25) (layer F.Cu) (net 65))
 (segment (start 149.046299 81.763501) (end 148.1963 82.6135) (width 0.25) (layer F.Cu) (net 66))
 (segment (start 149.561299 81.248501) (end 149.046299 81.763501) (width 0.25) (layer F.Cu) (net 66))
 (segment (start 149.561299 73.095101) (end 149.561299 81.248501) (width 0.25) (layer F.Cu) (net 66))
 (segment (start 151.638 71.0184) (end 149.561299 73.095101) (width 0.25) (layer F.Cu) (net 66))
 (segment (start 151.638 70.866) (end 151.638 71.0184) (width 0.25) (layer F.Cu) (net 66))
 (segment (start 154.178 76.6318) (end 150.7363 80.0735) (width 0.25) (layer F.Cu) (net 67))
 (segment (start 154.178 70.866) (end 154.178 76.6318) (width 0.25) (layer F.Cu) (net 67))
 (segment (start 151.586299 81.763501) (end 150.7363 82.6135) (width 0.25) (layer F.Cu) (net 68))
 (segment (start 151.911301 81.438499) (end 151.586299 81.763501) (width 0.25) (layer F.Cu) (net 68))
 (segment (start 151.911301 79.699497) (end 151.911301 81.438499) (width 0.25) (layer F.Cu) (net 68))
 (segment (start 156.718 74.892798) (end 151.911301 79.699497) (width 0.25) (layer F.Cu) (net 68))
 (segment (start 156.718 70.866) (end 156.718 74.892798) (width 0.25) (layer F.Cu) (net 68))
 (segment (start 153.2763 80.017289) (end 153.2763 80.0735) (width 0.25) (layer F.Cu) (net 69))
 (segment (start 159.258 70.866) (end 159.258 74.035589) (width 0.25) (layer F.Cu) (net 69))
 (segment (start 159.258 74.035589) (end 153.2763 80.017289) (width 0.25) (layer F.Cu) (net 69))
 (segment (start 154.126299 81.763501) (end 153.2763 82.6135) (width 0.25) (layer F.Cu) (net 70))
 (segment (start 154.451301 81.438499) (end 154.126299 81.763501) (width 0.25) (layer F.Cu) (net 70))
 (segment (start 154.451301 79.478699) (end 154.451301 81.438499) (width 0.25) (layer F.Cu) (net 70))
 (segment (start 161.798 72.132) (end 154.451301 79.478699) (width 0.25) (layer F.Cu) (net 70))
 (segment (start 161.798 70.866) (end 161.798 72.132) (width 0.25) (layer F.Cu) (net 70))
 (segment (start 155.8163 79.5401) (end 155.8163 80.0735) (width 0.25) (layer F.Cu) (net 71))
 (segment (start 164.338 71.0184) (end 155.8163 79.5401) (width 0.25) (layer F.Cu) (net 71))
 (segment (start 164.338 70.866) (end 164.338 71.0184) (width 0.25) (layer F.Cu) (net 71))
 (segment (start 156.666299 81.763501) (end 155.8163 82.6135) (width 0.25) (layer F.Cu) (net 72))
 (segment (start 156.991301 81.438499) (end 156.666299 81.763501) (width 0.25) (layer F.Cu) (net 72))
 (segment (start 158.730303 81.438499) (end 156.991301 81.438499) (width 0.25) (layer F.Cu) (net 72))
 (segment (start 159.531301 80.637501) (end 158.730303 81.438499) (width 0.25) (layer F.Cu) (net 72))
 (segment (start 159.531301 79.478699) (end 159.531301 80.637501) (width 0.25) (layer F.Cu) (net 72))
 (segment (start 166.878 72.132) (end 159.531301 79.478699) (width 0.25) (layer F.Cu) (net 72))
 (segment (start 166.878 70.866) (end 166.878 72.132) (width 0.25) (layer F.Cu) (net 72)))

